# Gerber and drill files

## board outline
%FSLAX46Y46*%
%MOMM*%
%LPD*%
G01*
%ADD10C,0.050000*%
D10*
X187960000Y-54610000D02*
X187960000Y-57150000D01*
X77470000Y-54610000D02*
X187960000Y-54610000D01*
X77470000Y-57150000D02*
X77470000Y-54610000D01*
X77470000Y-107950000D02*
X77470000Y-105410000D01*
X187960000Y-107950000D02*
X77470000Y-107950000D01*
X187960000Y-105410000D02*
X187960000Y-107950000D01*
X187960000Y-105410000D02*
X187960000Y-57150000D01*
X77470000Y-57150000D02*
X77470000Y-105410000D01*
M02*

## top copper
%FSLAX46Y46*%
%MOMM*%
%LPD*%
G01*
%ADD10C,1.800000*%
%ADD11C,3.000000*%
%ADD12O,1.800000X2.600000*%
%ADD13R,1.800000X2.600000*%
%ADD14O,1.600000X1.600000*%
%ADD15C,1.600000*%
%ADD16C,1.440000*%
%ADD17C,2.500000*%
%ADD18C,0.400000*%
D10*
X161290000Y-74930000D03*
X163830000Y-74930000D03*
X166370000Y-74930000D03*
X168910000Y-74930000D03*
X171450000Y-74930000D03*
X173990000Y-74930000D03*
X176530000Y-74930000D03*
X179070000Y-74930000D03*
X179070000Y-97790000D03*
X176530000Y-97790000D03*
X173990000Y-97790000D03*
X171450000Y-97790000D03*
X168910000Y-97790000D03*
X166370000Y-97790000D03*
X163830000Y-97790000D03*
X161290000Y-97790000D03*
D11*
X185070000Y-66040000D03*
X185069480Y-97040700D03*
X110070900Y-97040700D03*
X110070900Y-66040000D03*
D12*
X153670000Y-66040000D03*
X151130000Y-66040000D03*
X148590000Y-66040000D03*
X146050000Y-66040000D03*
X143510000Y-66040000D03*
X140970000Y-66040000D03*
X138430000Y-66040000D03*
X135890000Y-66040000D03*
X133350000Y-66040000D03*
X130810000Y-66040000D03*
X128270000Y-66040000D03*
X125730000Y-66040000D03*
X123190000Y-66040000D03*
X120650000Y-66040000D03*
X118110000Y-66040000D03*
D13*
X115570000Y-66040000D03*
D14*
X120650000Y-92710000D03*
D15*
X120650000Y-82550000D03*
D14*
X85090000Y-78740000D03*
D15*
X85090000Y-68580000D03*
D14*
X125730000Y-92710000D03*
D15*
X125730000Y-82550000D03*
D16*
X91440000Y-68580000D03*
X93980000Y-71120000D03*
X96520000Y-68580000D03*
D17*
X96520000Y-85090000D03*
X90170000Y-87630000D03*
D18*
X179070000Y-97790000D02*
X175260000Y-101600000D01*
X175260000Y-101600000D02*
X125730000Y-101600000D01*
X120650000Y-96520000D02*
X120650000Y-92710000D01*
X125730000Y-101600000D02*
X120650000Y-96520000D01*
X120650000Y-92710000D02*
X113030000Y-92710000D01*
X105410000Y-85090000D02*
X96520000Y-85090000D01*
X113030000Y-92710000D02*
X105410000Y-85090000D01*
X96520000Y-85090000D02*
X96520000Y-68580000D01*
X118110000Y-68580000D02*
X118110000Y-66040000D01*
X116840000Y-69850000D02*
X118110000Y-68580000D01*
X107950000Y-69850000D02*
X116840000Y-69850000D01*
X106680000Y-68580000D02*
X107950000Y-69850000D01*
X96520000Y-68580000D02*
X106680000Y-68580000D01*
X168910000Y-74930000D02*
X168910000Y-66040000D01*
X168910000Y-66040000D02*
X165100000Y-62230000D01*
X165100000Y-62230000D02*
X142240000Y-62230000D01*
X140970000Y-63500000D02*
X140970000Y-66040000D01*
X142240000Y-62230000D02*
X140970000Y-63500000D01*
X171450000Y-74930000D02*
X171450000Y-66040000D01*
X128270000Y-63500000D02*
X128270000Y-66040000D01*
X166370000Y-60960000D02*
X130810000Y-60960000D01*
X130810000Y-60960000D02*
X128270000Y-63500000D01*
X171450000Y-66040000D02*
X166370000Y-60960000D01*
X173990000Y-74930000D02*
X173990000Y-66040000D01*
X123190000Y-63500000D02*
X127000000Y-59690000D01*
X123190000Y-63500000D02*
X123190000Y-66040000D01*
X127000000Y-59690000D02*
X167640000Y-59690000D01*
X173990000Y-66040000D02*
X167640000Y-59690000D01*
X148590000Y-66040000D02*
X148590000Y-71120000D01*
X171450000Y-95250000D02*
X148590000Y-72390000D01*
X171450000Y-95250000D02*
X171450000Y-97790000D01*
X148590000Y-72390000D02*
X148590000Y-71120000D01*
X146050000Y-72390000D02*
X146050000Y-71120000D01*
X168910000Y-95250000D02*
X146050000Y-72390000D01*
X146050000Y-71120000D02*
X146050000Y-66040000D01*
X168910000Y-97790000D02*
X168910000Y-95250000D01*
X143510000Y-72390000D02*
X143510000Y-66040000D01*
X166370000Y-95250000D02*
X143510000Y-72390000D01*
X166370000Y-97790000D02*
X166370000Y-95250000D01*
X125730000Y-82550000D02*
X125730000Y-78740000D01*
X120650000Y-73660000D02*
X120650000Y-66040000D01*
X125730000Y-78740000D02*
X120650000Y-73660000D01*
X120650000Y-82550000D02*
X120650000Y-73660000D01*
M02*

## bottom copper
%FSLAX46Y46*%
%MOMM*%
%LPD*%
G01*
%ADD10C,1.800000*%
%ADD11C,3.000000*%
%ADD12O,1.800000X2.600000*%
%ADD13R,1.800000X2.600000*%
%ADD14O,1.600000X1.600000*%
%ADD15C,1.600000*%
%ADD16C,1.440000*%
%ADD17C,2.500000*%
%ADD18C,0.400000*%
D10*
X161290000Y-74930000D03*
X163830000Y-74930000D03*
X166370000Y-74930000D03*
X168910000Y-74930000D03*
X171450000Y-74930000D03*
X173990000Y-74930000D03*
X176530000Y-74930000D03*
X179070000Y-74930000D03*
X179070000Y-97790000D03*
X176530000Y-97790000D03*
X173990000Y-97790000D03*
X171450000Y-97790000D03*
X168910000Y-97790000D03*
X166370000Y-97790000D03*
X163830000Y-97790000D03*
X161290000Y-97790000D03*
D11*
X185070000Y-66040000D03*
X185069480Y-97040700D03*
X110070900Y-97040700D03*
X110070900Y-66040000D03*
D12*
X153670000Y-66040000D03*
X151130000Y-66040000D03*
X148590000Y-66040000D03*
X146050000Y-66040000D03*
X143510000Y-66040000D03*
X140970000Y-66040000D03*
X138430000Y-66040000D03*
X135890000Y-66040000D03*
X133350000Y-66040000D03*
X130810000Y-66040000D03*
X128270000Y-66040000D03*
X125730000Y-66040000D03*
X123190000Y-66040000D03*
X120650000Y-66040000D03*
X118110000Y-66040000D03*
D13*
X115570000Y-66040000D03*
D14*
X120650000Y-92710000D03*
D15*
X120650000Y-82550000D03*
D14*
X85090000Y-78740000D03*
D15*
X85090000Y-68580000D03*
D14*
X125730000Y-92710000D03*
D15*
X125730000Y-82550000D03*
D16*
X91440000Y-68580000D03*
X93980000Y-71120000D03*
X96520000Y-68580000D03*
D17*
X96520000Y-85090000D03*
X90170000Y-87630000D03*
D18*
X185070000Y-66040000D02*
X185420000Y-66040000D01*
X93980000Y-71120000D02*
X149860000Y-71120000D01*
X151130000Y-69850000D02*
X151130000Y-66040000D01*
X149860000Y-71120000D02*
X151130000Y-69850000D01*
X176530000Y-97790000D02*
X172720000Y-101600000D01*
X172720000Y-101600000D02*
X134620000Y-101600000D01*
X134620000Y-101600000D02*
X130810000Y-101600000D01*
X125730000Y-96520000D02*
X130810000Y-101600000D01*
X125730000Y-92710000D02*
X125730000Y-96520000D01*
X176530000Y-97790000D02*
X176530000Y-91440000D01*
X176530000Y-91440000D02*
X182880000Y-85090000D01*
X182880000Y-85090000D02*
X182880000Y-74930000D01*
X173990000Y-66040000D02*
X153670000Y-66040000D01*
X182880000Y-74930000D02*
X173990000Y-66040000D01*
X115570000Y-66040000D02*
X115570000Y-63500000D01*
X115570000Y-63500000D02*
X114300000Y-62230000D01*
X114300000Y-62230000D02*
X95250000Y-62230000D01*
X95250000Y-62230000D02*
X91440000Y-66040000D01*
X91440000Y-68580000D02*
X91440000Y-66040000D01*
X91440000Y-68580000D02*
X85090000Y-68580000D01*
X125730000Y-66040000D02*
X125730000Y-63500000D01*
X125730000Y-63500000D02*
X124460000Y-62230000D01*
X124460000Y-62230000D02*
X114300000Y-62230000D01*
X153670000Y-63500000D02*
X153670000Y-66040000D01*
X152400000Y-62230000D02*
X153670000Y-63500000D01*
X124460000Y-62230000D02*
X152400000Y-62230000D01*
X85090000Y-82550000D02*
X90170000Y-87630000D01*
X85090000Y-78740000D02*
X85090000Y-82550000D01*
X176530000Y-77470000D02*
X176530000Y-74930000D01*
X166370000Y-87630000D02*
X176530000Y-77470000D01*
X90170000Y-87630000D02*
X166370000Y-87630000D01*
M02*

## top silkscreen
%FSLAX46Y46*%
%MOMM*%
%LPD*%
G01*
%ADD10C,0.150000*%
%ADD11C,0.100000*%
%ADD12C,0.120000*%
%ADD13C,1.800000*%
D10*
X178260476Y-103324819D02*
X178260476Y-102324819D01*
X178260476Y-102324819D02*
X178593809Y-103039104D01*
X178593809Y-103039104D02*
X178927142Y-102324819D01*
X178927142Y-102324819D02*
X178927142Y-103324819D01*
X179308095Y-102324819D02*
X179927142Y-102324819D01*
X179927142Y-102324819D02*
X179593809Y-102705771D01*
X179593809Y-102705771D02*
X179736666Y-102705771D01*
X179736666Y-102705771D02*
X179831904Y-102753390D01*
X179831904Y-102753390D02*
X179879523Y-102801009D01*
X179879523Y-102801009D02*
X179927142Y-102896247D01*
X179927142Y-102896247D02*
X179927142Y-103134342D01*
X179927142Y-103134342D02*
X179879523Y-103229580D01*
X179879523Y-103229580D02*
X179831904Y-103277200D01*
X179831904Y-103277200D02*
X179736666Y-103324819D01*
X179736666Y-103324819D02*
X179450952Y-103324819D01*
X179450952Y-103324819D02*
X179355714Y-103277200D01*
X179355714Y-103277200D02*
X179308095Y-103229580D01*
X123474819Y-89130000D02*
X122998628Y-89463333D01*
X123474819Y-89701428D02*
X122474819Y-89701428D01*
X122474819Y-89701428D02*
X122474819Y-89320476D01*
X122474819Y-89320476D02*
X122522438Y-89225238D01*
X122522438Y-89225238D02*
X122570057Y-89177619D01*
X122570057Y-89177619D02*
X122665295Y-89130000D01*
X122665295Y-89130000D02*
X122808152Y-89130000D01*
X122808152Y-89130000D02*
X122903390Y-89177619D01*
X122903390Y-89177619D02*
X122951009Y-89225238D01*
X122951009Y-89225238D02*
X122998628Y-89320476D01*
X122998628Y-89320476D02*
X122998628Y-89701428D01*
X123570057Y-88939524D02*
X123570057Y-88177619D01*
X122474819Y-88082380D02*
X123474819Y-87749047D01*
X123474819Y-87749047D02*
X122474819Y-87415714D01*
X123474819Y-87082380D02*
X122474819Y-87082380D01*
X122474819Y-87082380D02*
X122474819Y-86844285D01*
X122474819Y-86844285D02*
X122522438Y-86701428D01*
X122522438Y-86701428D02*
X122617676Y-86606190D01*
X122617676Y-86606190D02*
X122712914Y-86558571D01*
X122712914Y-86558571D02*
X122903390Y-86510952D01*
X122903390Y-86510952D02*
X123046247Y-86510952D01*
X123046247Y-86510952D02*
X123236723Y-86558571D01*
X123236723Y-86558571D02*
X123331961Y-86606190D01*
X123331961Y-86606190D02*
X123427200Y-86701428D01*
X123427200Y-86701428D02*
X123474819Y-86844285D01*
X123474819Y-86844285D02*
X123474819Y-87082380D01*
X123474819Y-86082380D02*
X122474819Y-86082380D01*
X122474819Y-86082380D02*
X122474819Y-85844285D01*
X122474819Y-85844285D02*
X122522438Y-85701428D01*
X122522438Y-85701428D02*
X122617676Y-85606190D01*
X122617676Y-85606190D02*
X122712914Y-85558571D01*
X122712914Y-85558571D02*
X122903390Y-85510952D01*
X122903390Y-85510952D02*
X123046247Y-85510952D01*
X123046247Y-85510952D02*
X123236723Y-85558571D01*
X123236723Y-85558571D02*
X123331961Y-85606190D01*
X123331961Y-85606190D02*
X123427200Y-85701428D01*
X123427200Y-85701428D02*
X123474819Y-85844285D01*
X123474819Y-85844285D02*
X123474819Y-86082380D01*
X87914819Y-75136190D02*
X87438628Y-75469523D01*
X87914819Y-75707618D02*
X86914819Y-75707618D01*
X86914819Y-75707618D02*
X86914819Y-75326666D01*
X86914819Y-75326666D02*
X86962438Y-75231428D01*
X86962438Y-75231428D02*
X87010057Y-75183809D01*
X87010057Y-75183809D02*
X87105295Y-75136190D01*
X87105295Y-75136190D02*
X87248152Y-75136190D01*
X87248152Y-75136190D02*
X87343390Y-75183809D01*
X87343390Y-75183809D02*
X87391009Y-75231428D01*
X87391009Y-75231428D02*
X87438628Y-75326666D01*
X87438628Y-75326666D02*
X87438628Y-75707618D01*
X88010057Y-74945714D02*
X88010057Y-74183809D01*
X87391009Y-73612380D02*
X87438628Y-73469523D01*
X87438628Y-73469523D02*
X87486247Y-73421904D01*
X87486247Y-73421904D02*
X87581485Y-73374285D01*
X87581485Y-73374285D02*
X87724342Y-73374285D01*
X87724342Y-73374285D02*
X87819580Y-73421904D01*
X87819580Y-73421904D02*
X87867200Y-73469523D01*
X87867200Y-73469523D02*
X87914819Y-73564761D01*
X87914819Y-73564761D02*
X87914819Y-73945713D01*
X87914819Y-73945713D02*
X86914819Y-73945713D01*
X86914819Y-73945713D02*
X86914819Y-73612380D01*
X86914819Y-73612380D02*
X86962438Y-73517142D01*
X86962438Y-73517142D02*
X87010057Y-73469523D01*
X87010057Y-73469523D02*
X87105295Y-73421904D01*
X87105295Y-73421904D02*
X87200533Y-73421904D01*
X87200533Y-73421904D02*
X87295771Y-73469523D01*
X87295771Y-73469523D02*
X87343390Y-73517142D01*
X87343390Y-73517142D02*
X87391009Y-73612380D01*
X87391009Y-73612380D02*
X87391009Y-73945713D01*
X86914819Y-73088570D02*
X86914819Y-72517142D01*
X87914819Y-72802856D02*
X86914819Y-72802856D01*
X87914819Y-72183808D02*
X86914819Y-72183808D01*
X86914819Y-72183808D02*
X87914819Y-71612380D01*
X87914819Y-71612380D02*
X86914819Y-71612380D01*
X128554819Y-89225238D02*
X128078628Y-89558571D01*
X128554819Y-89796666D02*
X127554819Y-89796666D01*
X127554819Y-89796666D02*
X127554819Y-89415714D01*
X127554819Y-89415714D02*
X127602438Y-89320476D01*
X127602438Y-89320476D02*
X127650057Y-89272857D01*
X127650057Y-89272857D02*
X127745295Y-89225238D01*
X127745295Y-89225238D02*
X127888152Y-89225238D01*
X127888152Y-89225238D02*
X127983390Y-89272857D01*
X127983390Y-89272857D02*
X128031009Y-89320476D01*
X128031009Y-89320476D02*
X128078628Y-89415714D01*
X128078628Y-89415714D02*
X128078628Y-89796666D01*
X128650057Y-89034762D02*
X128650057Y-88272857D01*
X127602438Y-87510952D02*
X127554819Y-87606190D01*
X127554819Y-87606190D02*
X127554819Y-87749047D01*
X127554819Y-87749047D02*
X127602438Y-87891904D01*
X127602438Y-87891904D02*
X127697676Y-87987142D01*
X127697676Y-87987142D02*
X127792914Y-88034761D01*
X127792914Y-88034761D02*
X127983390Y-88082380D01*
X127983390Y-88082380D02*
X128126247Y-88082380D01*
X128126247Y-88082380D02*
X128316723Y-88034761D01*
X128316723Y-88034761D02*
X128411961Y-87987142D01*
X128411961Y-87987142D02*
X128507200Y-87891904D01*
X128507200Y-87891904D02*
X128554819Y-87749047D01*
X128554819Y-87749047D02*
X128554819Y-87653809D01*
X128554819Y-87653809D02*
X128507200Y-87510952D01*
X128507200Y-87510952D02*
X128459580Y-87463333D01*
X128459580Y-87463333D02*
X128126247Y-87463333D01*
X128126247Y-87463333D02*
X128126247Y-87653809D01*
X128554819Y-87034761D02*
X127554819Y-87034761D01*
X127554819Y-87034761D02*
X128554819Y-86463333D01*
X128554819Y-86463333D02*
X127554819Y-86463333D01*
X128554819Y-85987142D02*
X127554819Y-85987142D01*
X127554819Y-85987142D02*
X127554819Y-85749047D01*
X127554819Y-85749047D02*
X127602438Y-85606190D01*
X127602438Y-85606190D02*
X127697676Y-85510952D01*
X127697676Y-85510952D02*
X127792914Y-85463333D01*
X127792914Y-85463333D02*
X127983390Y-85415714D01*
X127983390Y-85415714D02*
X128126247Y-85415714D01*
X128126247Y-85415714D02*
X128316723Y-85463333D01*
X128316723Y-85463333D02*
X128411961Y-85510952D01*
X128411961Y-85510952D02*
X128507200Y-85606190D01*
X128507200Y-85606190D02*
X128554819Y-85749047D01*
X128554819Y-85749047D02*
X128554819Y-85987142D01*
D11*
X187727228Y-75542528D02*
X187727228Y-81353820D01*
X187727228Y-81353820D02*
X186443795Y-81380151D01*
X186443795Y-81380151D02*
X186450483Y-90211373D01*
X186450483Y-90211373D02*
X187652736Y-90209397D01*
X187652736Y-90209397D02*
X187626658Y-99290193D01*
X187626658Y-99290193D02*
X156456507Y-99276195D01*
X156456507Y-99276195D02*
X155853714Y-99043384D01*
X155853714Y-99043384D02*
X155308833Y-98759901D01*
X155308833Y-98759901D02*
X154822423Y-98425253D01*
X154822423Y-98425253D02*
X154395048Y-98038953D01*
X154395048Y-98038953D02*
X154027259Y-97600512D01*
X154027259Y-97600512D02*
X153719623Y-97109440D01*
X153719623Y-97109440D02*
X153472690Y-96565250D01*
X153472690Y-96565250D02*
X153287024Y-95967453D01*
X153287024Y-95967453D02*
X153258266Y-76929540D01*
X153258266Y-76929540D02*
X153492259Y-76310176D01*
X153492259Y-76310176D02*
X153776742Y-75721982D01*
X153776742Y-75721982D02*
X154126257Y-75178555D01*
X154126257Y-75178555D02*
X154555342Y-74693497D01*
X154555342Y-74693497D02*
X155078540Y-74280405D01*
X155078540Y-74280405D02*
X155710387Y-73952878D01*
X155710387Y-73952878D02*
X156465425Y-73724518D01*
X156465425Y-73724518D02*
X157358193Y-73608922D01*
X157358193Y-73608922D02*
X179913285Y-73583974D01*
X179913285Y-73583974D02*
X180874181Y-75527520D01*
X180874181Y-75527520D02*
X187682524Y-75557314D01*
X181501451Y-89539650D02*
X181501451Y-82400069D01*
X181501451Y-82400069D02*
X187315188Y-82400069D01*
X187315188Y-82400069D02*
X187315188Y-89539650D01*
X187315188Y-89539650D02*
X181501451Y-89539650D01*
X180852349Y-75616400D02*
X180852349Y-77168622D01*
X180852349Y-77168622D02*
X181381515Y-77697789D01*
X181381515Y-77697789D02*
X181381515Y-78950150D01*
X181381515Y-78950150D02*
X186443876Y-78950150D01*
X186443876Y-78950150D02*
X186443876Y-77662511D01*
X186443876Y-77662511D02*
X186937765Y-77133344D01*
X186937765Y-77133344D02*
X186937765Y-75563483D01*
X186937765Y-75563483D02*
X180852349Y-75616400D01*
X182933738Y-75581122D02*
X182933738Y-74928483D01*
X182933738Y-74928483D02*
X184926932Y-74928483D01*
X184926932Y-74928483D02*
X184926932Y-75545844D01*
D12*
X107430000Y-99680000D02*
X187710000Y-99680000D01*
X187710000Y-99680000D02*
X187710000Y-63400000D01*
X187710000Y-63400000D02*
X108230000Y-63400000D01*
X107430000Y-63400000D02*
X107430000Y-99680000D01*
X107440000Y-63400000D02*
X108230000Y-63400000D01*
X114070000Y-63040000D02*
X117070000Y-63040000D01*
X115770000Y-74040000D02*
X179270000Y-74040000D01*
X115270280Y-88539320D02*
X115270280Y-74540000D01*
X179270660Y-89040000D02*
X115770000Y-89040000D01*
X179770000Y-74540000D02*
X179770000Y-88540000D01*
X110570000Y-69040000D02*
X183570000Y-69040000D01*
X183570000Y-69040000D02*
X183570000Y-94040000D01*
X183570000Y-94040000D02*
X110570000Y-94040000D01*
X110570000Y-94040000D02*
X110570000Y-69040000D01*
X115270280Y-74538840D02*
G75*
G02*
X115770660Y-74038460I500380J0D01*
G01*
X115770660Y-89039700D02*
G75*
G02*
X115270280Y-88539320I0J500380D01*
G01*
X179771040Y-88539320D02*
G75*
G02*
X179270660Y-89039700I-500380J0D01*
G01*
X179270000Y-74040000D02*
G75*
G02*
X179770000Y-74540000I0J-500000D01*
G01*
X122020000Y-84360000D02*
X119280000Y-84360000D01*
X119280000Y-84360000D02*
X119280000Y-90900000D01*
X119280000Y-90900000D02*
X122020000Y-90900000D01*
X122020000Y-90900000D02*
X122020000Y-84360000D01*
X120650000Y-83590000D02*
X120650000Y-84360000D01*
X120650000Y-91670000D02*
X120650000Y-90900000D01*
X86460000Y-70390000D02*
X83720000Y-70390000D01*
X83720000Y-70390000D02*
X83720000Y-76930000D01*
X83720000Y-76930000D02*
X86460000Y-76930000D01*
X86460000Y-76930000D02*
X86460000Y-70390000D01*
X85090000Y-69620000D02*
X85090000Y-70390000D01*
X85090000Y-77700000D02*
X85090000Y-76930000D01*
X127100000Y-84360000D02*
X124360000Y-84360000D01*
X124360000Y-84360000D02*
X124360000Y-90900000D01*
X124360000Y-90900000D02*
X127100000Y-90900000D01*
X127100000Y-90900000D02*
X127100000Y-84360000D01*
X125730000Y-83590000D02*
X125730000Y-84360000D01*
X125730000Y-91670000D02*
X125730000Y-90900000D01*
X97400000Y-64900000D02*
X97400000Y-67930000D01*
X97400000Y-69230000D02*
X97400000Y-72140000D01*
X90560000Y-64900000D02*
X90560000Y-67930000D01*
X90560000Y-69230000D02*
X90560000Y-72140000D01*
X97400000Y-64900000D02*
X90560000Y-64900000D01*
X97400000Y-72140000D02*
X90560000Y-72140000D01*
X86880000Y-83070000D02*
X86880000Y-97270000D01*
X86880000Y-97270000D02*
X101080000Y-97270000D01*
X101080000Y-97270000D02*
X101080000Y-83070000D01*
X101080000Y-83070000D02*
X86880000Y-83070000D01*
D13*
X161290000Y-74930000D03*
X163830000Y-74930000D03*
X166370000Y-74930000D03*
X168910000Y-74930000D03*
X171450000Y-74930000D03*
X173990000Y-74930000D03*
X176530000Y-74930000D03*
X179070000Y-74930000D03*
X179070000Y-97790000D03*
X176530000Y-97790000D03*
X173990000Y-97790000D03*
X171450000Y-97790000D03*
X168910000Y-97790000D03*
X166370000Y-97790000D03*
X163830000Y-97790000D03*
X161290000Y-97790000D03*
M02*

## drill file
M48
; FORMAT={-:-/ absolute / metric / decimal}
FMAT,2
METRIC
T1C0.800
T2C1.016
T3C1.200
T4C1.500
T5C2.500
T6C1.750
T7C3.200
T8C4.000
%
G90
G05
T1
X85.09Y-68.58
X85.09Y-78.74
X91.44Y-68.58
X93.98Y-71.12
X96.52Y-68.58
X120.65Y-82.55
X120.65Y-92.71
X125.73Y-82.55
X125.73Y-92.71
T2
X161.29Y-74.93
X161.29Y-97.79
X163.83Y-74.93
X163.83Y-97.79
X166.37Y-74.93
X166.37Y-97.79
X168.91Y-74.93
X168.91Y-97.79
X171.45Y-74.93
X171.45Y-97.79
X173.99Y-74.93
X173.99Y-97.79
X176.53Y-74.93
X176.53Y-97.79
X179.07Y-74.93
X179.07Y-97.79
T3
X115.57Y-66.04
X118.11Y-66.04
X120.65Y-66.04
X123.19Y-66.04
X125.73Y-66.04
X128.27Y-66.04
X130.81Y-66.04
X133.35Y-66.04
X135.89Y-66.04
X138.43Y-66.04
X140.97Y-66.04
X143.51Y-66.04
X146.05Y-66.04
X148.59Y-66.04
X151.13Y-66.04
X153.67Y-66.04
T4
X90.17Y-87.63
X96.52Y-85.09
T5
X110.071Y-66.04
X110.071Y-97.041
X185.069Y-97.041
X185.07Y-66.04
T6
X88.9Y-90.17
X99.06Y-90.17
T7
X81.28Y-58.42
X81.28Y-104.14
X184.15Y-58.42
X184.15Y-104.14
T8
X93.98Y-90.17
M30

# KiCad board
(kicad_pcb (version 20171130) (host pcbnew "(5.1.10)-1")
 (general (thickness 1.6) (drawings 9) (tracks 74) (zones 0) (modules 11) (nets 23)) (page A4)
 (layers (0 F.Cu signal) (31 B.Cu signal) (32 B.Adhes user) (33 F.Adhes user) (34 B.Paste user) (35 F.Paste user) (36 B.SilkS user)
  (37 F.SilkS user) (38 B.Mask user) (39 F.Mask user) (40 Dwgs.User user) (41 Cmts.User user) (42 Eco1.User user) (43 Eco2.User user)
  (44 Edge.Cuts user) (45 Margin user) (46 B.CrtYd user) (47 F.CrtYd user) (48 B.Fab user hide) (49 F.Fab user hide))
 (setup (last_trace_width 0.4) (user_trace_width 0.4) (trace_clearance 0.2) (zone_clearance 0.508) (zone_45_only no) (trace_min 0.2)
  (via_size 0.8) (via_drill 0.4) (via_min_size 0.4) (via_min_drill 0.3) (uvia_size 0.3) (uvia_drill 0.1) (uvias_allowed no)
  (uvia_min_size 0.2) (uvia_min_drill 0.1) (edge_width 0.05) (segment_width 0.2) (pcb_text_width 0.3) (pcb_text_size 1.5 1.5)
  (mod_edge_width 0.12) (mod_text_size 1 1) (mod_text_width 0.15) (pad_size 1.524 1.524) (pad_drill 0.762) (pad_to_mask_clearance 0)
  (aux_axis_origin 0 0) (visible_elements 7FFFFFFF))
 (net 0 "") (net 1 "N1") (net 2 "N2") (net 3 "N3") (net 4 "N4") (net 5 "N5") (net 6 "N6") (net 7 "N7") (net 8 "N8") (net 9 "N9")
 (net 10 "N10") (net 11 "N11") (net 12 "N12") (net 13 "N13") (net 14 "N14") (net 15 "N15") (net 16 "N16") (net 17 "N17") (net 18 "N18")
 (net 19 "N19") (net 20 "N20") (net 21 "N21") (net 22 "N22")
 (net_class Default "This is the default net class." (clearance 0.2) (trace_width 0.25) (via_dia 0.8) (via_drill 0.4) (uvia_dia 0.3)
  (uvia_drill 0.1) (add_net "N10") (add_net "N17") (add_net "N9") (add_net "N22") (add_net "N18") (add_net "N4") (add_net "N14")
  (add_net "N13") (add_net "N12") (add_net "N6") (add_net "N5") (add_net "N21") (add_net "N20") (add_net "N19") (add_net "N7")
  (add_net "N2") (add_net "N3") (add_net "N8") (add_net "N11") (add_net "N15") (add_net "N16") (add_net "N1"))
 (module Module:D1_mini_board (layer F.Cu) (at 171.45 86.36 90)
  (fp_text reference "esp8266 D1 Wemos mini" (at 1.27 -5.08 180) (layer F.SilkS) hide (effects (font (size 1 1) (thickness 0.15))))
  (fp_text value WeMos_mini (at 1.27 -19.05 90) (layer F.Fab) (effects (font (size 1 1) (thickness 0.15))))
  (fp_line (start 10.817472 16.277228) (end 5.00618 16.277228) (layer F.SilkS) (width 0.1))
  (fp_line (start 5.00618 16.277228) (end 4.979849 14.993795) (layer F.SilkS) (width 0.1))
  (fp_line (start 4.979849 14.993795) (end -3.851373 15.000483) (layer F.SilkS) (width 0.1))
  (fp_line (start -3.851373 15.000483) (end -3.849397 16.202736) (layer F.SilkS) (width 0.1))
  (fp_line (start -3.849397 16.202736) (end -12.930193 16.176658) (layer F.SilkS) (width 0.1))
  (fp_line (start -12.930193 16.176658) (end -12.916195 -14.993493) (layer F.SilkS) (width 0.1))
  (fp_line (start -12.916195 -14.993493) (end -12.683384 -15.596286) (layer F.SilkS) (width 0.1))
  (fp_line (start -12.683384 -15.596286) (end -12.399901 -16.141167) (layer F.SilkS) (width 0.1))
  (fp_line (start -12.399901 -16.141167) (end -12.065253 -16.627577) (layer F.SilkS) (width 0.1))
  (fp_line (start -12.065253 -16.627577) (end -11.678953 -17.054952) (layer F.SilkS) (width 0.1))
  (fp_line (start -11.678953 -17.054952) (end -11.240512 -17.422741) (layer F.SilkS) (width 0.1))
  (fp_line (start -11.240512 -17.422741) (end -10.74944 -17.730377) (layer F.SilkS) (width 0.1))
  (fp_line (start -10.74944 -17.730377) (end -10.20525 -17.97731) (layer F.SilkS) (width 0.1))
  (fp_line (start -10.20525 -17.97731) (end -9.607453 -18.162976) (layer F.SilkS) (width 0.1))
  (fp_line (start -9.607453 -18.162976) (end 9.43046 -18.191734) (layer F.SilkS) (width 0.1))
  (fp_line (start 9.43046 -18.191734) (end 10.049824 -17.957741) (layer F.SilkS) (width 0.1))
  (fp_line (start 10.049824 -17.957741) (end 10.638018 -17.673258) (layer F.SilkS) (width 0.1))
  (fp_line (start 10.638018 -17.673258) (end 11.181445 -17.323743) (layer F.SilkS) (width 0.1))
  (fp_line (start 11.181445 -17.323743) (end 11.666503 -16.894658) (layer F.SilkS) (width 0.1))
  (fp_line (start 11.666503 -16.894658) (end 12.079595 -16.37146) (layer F.SilkS) (width 0.1))
  (fp_line (start 12.079595 -16.37146) (end 12.407122 -15.739613) (layer F.SilkS) (width 0.1))
  (fp_line (start 12.407122 -15.739613) (end 12.635482 -14.984575) (layer F.SilkS) (width 0.1))
  (fp_line (start 12.635482 -14.984575) (end 12.751078 -14.091807) (layer F.SilkS) (width 0.1))
  (fp_line (start 12.751078 -14.091807) (end 12.776026 8.463285) (layer F.SilkS) (width 0.1))
  (fp_line (start 12.776026 8.463285) (end 10.83248 9.424181) (layer F.SilkS) (width 0.1))
  (fp_line (start 10.83248 9.424181) (end 10.802686 16.232524) (layer F.SilkS) (width 0.1))
  (fp_line (start -3.17965 10.051451) (end 3.959931 10.051451) (layer F.SilkS) (width 0.1))
  (fp_line (start 3.959931 10.051451) (end 3.959931 15.865188) (layer F.SilkS) (width 0.1))
  (fp_line (start 3.959931 15.865188) (end -3.17965 15.865188) (layer F.SilkS) (width 0.1))
  (fp_line (start -3.17965 15.865188) (end -3.17965 10.051451) (layer F.SilkS) (width 0.1))
  (fp_line (start 10.7436 9.402349) (end 9.191378 9.402349) (layer F.SilkS) (width 0.1))
  (fp_line (start 9.191378 9.402349) (end 8.662211 9.931515) (layer F.SilkS) (width 0.1))
  (fp_line (start 8.662211 9.931515) (end 7.40985 9.931515) (layer F.SilkS) (width 0.1))
  (fp_line (start 7.40985 9.931515) (end 7.40985 14.993876) (layer F.SilkS) (width 0.1))
  (fp_line (start 7.40985 14.993876) (end 8.697489 14.993876) (layer F.SilkS) (width 0.1))
  (fp_line (start 8.697489 14.993876) (end 9.226656 15.487765) (layer F.SilkS) (width 0.1))
  (fp_line (start 9.226656 15.487765) (end 10.796517 15.487765) (layer F.SilkS) (width 0.1))
  (fp_line (start 10.796517 15.487765) (end 10.7436 9.402349) (layer F.SilkS) (width 0.1))
  (fp_line (start 10.778878 11.483738) (end 11.431517 11.483738) (layer F.SilkS) (width 0.1))
  (fp_line (start 11.431517 11.483738) (end 11.431517 13.476932) (layer F.SilkS) (width 0.1))
  (fp_line (start 11.431517 13.476932) (end 10.814156 13.476932) (layer F.SilkS) (width 0.1))
  (pad 9 thru_hole circle (at 11.43 -10.16 90) (size 1.8 1.8) (drill 1.016) (layers *.Cu *.Mask F.SilkS) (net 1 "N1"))
  (pad 10 thru_hole circle (at 11.43 -7.62 90) (size 1.8 1.8) (drill 1.016) (layers *.Cu *.Mask F.SilkS) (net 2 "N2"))
  (pad 11 thru_hole circle (at 11.43 -5.08 90) (size 1.8 1.8) (drill 1.016) (layers *.Cu *.Mask F.SilkS) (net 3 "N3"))
  (pad 12 thru_hole circle (at 11.43 -2.54 90) (size 1.8 1.8) (drill 1.016) (layers *.Cu *.Mask F.SilkS) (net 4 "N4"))
  (pad 13 thru_hole circle (at 11.43 0 90) (size 1.8 1.8) (drill 1.016) (layers *.Cu *.Mask F.SilkS) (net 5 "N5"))
  (pad 14 thru_hole circle (at 11.43 2.54 90) (size 1.8 1.8) (drill 1.016) (layers *.Cu *.Mask F.SilkS) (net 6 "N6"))
  (pad 15 thru_hole circle (at 11.43 5.08 90) (size 1.8 1.8) (drill 1.016) (layers *.Cu *.Mask F.SilkS) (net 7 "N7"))
  (pad 16 thru_hole circle (at 11.43 7.62 90) (size 1.8 1.8) (drill 1.016) (layers *.Cu *.Mask F.SilkS) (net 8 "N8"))
  (pad 1 thru_hole circle (at -11.43 7.62 90) (size 1.8 1.8) (drill 1.016) (layers *.Cu *.Mask F.SilkS) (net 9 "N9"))
  (pad 2 thru_hole circle (at -11.43 5.08 90) (size 1.8 1.8) (drill 1.016) (layers *.Cu *.Mask F.SilkS) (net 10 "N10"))
  (pad 3 thru_hole circle (at -11.43 2.54 90) (size 1.8 1.8) (drill 1.016) (layers *.Cu *.Mask F.SilkS) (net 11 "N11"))
  (pad 4 thru_hole circle (at -11.43 0 90) (size 1.8 1.8) (drill 1.016) (layers *.Cu *.Mask F.SilkS) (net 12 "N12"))
  (pad 5 thru_hole circle (at -11.43 -2.54 90) (size 1.8 1.8) (drill 1.016) (layers *.Cu *.Mask F.SilkS) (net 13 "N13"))
  (pad 6 thru_hole circle (at -11.43 -5.08 90) (size 1.8 1.8) (drill 1.016) (layers *.Cu *.Mask F.SilkS) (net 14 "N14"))
  (pad 7 thru_hole circle (at -11.43 -7.62 90) (size 1.8 1.8) (drill 1.016) (layers *.Cu *.Mask F.SilkS) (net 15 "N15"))
  (pad 8 thru_hole circle (at -11.43 -10.16 90) (size 1.8 1.8) (drill 1.016) (layers *.Cu *.Mask F.SilkS) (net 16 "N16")))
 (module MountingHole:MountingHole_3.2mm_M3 (layer F.Cu) (at 184.15 104.14)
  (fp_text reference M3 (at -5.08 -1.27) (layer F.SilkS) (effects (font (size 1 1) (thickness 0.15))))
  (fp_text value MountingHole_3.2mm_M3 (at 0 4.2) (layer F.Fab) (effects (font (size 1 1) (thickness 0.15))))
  (pad 1 np_thru_hole circle (at 0 0) (size 3.2 3.2) (drill 3.2) (layers *.Cu *.Mask)))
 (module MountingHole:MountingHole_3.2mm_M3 (layer F.Cu) (at 81.28 104.14)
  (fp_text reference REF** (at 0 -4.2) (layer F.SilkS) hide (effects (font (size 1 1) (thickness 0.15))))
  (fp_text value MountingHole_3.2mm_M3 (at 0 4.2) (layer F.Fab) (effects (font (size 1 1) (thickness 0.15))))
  (pad 1 np_thru_hole circle (at 0 0) (size 3.2 3.2) (drill 3.2) (layers *.Cu *.Mask)))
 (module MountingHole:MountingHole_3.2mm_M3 (layer F.Cu) (at 81.28 58.42)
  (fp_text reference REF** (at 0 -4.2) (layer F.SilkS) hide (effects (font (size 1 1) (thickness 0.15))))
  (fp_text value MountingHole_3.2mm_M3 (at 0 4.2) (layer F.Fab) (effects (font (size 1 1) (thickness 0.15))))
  (pad 1 np_thru_hole circle (at 0 0) (size 3.2 3.2) (drill 3.2) (layers *.Cu *.Mask)))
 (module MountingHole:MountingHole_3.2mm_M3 (layer F.Cu) (at 184.15 58.42)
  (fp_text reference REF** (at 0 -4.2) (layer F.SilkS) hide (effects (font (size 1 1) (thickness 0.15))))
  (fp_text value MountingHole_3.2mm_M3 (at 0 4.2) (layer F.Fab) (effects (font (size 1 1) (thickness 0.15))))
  (pad 1 np_thru_hole circle (at 0 0) (size 3.2 3.2) (drill 3.2) (layers *.Cu *.Mask)))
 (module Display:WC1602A (layer F.Cu) (at 115.57 66.04)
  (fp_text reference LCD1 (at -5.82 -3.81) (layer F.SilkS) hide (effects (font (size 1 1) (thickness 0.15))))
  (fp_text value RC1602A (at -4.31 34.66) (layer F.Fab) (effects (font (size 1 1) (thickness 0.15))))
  (fp_line (start -8.14 33.64) (end 72.14 33.64) (layer F.SilkS) (width 0.12))
  (fp_line (start 72.14 33.64) (end 72.14 -2.64) (layer F.SilkS) (width 0.12))
  (fp_line (start 72.14 -2.64) (end -7.34 -2.64) (layer F.SilkS) (width 0.12))
  (fp_line (start -8.14 -2.64) (end -8.14 33.64) (layer F.SilkS) (width 0.12))
  (fp_line (start -8.13 -2.64) (end -7.34 -2.64) (layer F.SilkS) (width 0.12))
  (fp_line (start -1.5 -3) (end 1.5 -3) (layer F.SilkS) (width 0.12))
  (fp_line (start 0.2 8) (end 63.7 8) (layer F.SilkS) (width 0.12))
  (fp_line (start -0.29972 22.49932) (end -0.29972 8.5) (layer F.SilkS) (width 0.12))
  (fp_line (start 63.70066 23) (end 0.2 23) (layer F.SilkS) (width 0.12))
  (fp_line (start 64.2 8.5) (end 64.2 22.5) (layer F.SilkS) (width 0.12))
  (fp_line (start -5 3) (end 68 3) (layer F.SilkS) (width 0.12))
  (fp_line (start 68 3) (end 68 28) (layer F.SilkS) (width 0.12))
  (fp_line (start 68 28) (end -5 28) (layer F.SilkS) (width 0.12))
  (fp_line (start -5 28) (end -5 3) (layer F.SilkS) (width 0.12))
  (fp_arc (start 0.20066 8.49884) (end -0.29972 8.49884) (angle 90) (layer F.SilkS) (width 0.12))
  (fp_arc (start 0.20066 22.49932) (end 0.20066 22.9997) (angle 90) (layer F.SilkS) (width 0.12))
  (fp_arc (start 63.70066 22.49932) (end 64.20104 22.49932) (angle 90) (layer F.SilkS) (width 0.12))
  (fp_arc (start 63.7 8.5) (end 63.7 8) (angle 90) (layer F.SilkS) (width 0.12))
  (pad "" thru_hole circle (at 69.5 0) (size 3 3) (drill 2.5) (layers *.Cu *.Mask))
  (pad "" thru_hole circle (at 69.49948 31.0007) (size 3 3) (drill 2.5) (layers *.Cu *.Mask))
  (pad "" thru_hole circle (at -5.4991 31.0007) (size 3 3) (drill 2.5) (layers *.Cu *.Mask))
  (pad "" thru_hole circle (at -5.4991 0) (size 3 3) (drill 2.5) (layers *.Cu *.Mask))
  (pad 16 thru_hole oval (at 38.1 0) (size 1.8 2.6) (drill 1.2) (layers *.Cu *.Mask) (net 10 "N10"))
  (pad 15 thru_hole oval (at 35.56 0) (size 1.8 2.6) (drill 1.2) (layers *.Cu *.Mask) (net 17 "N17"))
  (pad 14 thru_hole oval (at 33.02 0) (size 1.8 2.6) (drill 1.2) (layers *.Cu *.Mask) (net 12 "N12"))
  (pad 13 thru_hole oval (at 30.48 0) (size 1.8 2.6) (drill 1.2) (layers *.Cu *.Mask) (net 13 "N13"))
  (pad 12 thru_hole oval (at 27.94 0) (size 1.8 2.6) (drill 1.2) (layers *.Cu *.Mask) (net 14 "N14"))
  (pad 11 thru_hole oval (at 25.4 0) (size 1.8 2.6) (drill 1.2) (layers *.Cu *.Mask) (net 4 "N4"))
  (pad 10 thru_hole oval (at 22.86 0) (size 1.8 2.6) (drill 1.2) (layers *.Cu *.Mask) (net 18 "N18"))
  (pad 9 thru_hole oval (at 20.32 0) (size 1.8 2.6) (drill 1.2) (layers *.Cu *.Mask) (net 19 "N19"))
  (pad 8 thru_hole oval (at 17.78 0) (size 1.8 2.6) (drill 1.2) (layers *.Cu *.Mask) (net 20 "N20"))
  (pad 7 thru_hole oval (at 15.24 0) (size 1.8 2.6) (drill 1.2) (layers *.Cu *.Mask) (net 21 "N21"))
  (pad 6 thru_hole oval (at 12.7 0) (size 1.8 2.6) (drill 1.2) (layers *.Cu *.Mask) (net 5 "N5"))
  (pad 5 thru_hole oval (at 10.16 0) (size 1.8 2.6) (drill 1.2) (layers *.Cu *.Mask) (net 10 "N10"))
  (pad 4 thru_hole oval (at 7.62 0) (size 1.8 2.6) (drill 1.2) (layers *.Cu *.Mask) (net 6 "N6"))
  (pad 3 thru_hole oval (at 5.08 0) (size 1.8 2.6) (drill 1.2) (layers *.Cu *.Mask) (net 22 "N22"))
  (pad 2 thru_hole oval (at 2.54 0) (size 1.8 2.6) (drill 1.2) (layers *.Cu *.Mask) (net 9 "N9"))
  (pad 1 thru_hole rect (at 0 0) (size 1.8 2.6) (drill 1.2) (layers *.Cu *.Mask) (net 10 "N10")))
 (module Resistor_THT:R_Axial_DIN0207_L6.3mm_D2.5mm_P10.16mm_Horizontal (layer F.Cu) (at 120.65 82.55 270)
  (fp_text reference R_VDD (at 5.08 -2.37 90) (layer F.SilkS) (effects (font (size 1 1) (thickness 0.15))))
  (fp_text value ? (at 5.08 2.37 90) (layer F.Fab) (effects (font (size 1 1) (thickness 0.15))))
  (fp_line (start 1.81 -1.37) (end 1.81 1.37) (layer F.SilkS) (width 0.12))
  (fp_line (start 1.81 1.37) (end 8.35 1.37) (layer F.SilkS) (width 0.12))
  (fp_line (start 8.35 1.37) (end 8.35 -1.37) (layer F.SilkS) (width 0.12))
  (fp_line (start 8.35 -1.37) (end 1.81 -1.37) (layer F.SilkS) (width 0.12))
  (fp_line (start 1.04 0) (end 1.81 0) (layer F.SilkS) (width 0.12))
  (fp_line (start 9.12 0) (end 8.35 0) (layer F.SilkS) (width 0.12))
  (pad 2 thru_hole oval (at 10.16 0 270) (size 1.6 1.6) (drill 0.8) (layers *.Cu *.Mask) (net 9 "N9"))
  (pad 1 thru_hole circle (at 0 0 270) (size 1.6 1.6) (drill 0.8) (layers *.Cu *.Mask) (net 22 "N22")))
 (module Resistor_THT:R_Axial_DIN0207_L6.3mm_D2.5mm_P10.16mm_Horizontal (layer F.Cu) (at 85.09 68.58 270)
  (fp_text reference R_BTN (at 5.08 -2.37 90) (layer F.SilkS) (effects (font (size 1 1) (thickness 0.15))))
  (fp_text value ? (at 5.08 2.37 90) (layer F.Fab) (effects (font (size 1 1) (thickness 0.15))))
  (fp_line (start 1.81 -1.37) (end 1.81 1.37) (layer F.SilkS) (width 0.12))
  (fp_line (start 1.81 1.37) (end 8.35 1.37) (layer F.SilkS) (width 0.12))
  (fp_line (start 8.35 1.37) (end 8.35 -1.37) (layer F.SilkS) (width 0.12))
  (fp_line (start 8.35 -1.37) (end 1.81 -1.37) (layer F.SilkS) (width 0.12))
  (fp_line (start 1.04 0) (end 1.81 0) (layer F.SilkS) (width 0.12))
  (fp_line (start 9.12 0) (end 8.35 0) (layer F.SilkS) (width 0.12))
  (pad 2 thru_hole oval (at 10.16 0 270) (size 1.6 1.6) (drill 0.8) (layers *.Cu *.Mask) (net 7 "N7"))
  (pad 1 thru_hole circle (at 0 0 270) (size 1.6 1.6) (drill 0.8) (layers *.Cu *.Mask) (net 10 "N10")))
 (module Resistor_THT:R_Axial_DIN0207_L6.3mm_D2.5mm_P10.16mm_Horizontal (layer F.Cu) (at 125.73 82.55 270)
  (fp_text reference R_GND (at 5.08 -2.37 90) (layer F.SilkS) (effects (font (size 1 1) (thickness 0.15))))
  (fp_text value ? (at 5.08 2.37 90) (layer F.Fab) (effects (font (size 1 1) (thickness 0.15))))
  (fp_line (start 1.81 -1.37) (end 1.81 1.37) (layer F.SilkS) (width 0.12))
  (fp_line (start 1.81 1.37) (end 8.35 1.37) (layer F.SilkS) (width 0.12))
  (fp_line (start 8.35 1.37) (end 8.35 -1.37) (layer F.SilkS) (width 0.12))
  (fp_line (start 8.35 -1.37) (end 1.81 -1.37) (layer F.SilkS) (width 0.12))
  (fp_line (start 1.04 0) (end 1.81 0) (layer F.SilkS) (width 0.12))
  (fp_line (start 9.12 0) (end 8.35 0) (layer F.SilkS) (width 0.12))
  (pad 2 thru_hole oval (at 10.16 0 270) (size 1.6 1.6) (drill 0.8) (layers *.Cu *.Mask) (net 10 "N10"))
  (pad 1 thru_hole circle (at 0 0 270) (size 1.6 1.6) (drill 0.8) (layers *.Cu *.Mask) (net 22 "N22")))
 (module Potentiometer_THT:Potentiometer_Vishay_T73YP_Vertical (layer F.Cu) (at 91.44 68.58 270)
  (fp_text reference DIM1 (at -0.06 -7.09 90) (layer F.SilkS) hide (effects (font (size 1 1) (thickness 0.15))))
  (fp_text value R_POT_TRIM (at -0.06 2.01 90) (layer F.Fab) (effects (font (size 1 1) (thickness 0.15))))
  (fp_line (start -3.68 -5.96) (end -0.65 -5.96) (layer F.SilkS) (width 0.12))
  (fp_line (start 0.65 -5.96) (end 3.56 -5.96) (layer F.SilkS) (width 0.12))
  (fp_line (start -3.68 0.88) (end -0.65 0.88) (layer F.SilkS) (width 0.12))
  (fp_line (start 0.65 0.88) (end 3.56 0.88) (layer F.SilkS) (width 0.12))
  (fp_line (start -3.68 -5.96) (end -3.68 0.88) (layer F.SilkS) (width 0.12))
  (fp_line (start 3.56 -5.96) (end 3.56 0.88) (layer F.SilkS) (width 0.12))
  (pad 1 thru_hole circle (at 0 0 270) (size 1.44 1.44) (drill 0.8) (layers *.Cu *.Mask) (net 10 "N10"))
  (pad 2 thru_hole circle (at 2.54 -2.54 270) (size 1.44 1.44) (drill 0.8) (layers *.Cu *.Mask) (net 17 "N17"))
  (pad 3 thru_hole circle (at 0 -5.08 270) (size 1.44 1.44) (drill 0.8) (layers *.Cu *.Mask) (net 9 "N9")))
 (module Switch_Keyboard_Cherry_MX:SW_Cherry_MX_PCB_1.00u (layer F.Cu) (at 93.98 90.17)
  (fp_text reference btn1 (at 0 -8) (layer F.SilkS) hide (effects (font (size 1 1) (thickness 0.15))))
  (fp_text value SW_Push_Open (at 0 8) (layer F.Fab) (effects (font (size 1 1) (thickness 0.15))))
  (fp_line (start -7.1 -7.1) (end -7.1 7.1) (layer F.SilkS) (width 0.12))
  (fp_line (start -7.1 7.1) (end 7.1 7.1) (layer F.SilkS) (width 0.12))
  (fp_line (start 7.1 7.1) (end 7.1 -7.1) (layer F.SilkS) (width 0.12))
  (fp_line (start 7.1 -7.1) (end -7.1 -7.1) (layer F.SilkS) (width 0.12))
  (pad "" np_thru_hole circle (at 5.08 0) (size 1.75 1.75) (drill 1.75) (layers *.Cu *.Mask))
  (pad "" np_thru_hole circle (at -5.08 0) (size 1.75 1.75) (drill 1.75) (layers *.Cu *.Mask))
  (pad "" np_thru_hole circle (at 0 0) (size 4 4) (drill 4) (layers *.Cu *.Mask))
  (pad 2 thru_hole circle (at 2.54 -5.08) (size 2.5 2.5) (drill 1.5) (layers *.Cu B.Mask) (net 9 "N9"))
  (pad 1 thru_hole circle (at -3.81 -2.54) (size 2.5 2.5) (drill 1.5) (layers *.Cu B.Mask) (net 7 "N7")))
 (gr_line (start 187.96 54.61) (end 187.96 57.15) (layer Edge.Cuts) (width 0.05))
 (gr_line (start 77.47 54.61) (end 187.96 54.61) (layer Edge.Cuts) (width 0.05))
 (gr_line (start 77.47 57.15) (end 77.47 54.61) (layer Edge.Cuts) (width 0.05))
 (gr_line (start 77.47 107.95) (end 77.47 105.41) (layer Edge.Cuts) (width 0.05))
 (gr_line (start 187.96 107.95) (end 77.47 107.95) (layer Edge.Cuts) (width 0.05))
 (gr_line (start 187.96 105.41) (end 187.96 107.95) (layer Edge.Cuts) (width 0.05))
 (gr_line (start 187.96 105.41) (end 187.96 57.15) (layer Edge.Cuts) (width 0.05))
 (gr_line (start 77.47 57.15) (end 77.47 105.41) (layer Edge.Cuts) (width 0.05))
 (segment (start 185.07 66.04) (end 185.42 66.04) (width 0.4) (layer B.Cu) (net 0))
 (segment (start 179.07 97.79) (end 175.26 101.6) (width 0.4) (layer F.Cu) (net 9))
 (segment (start 175.26 101.6) (end 125.73 101.6) (width 0.4) (layer F.Cu) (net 9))
 (segment (start 120.65 96.52) (end 120.65 92.71) (width 0.4) (layer F.Cu) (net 9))
 (segment (start 125.73 101.6) (end 120.65 96.52) (width 0.4) (layer F.Cu) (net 9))
 (segment (start 120.65 92.71) (end 113.03 92.71) (width 0.4) (layer F.Cu) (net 9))
 (segment (start 105.41 85.09) (end 96.52 85.09) (width 0.4) (layer F.Cu) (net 9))
 (segment (start 113.03 92.71) (end 105.41 85.09) (width 0.4) (layer F.Cu) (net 9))
 (segment (start 96.52 85.09) (end 96.52 68.58) (width 0.4) (layer F.Cu) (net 9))
 (segment (start 118.11 68.58) (end 118.11 66.04) (width 0.4) (layer F.Cu) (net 9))
 (segment (start 116.84 69.85) (end 118.11 68.58) (width 0.4) (layer F.Cu) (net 9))
 (segment (start 107.95 69.85) (end 116.84 69.85) (width 0.4) (layer F.Cu) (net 9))
 (segment (start 106.68 68.58) (end 107.95 69.85) (width 0.4) (layer F.Cu) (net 9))
 (segment (start 96.52 68.58) (end 106.68 68.58) (width 0.4) (layer F.Cu) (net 9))
 (segment (start 93.98 71.12) (end 149.86 71.12) (width 0.4) (layer B.Cu) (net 17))
 (segment (start 151.13 69.85) (end 151.13 66.04) (width 0.4) (layer B.Cu) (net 17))
 (segment (start 149.86 71.12) (end 151.13 69.85) (width 0.4) (layer B.Cu) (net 17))
 (segment (start 176.53 97.79) (end 172.72 101.6) (width 0.4) (layer B.Cu) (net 10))
 (segment (start 172.72 101.6) (end 134.62 101.6) (width 0.4) (layer B.Cu) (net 10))
 (segment (start 134.62 101.6) (end 130.81 101.6) (width 0.4) (layer B.Cu) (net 10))
 (segment (start 125.73 96.52) (end 130.81 101.6) (width 0.4) (layer B.Cu) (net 10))
 (segment (start 125.73 92.71) (end 125.73 96.52) (width 0.4) (layer B.Cu) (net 10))
 (segment (start 176.53 97.79) (end 176.53 91.44) (width 0.4) (layer B.Cu) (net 10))
 (segment (start 176.53 91.44) (end 182.88 85.09) (width 0.4) (layer B.Cu) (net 10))
 (segment (start 182.88 85.09) (end 182.88 74.93) (width 0.4) (layer B.Cu) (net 10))
 (segment (start 173.99 66.04) (end 153.67 66.04) (width 0.4) (layer B.Cu) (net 10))
 (segment (start 182.88 74.93) (end 173.99 66.04) (width 0.4) (layer B.Cu) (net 10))
 (segment (start 115.57 66.04) (end 115.57 63.5) (width 0.4) (layer B.Cu) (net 10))
 (segment (start 115.57 63.5) (end 114.3 62.23) (width 0.4) (layer B.Cu) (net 10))
 (segment (start 114.3 62.23) (end 95.25 62.23) (width 0.4) (layer B.Cu) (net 10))
 (segment (start 95.25 62.23) (end 91.44 66.04) (width 0.4) (layer B.Cu) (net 10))
 (segment (start 91.44 68.58) (end 91.44 66.04) (width 0.4) (layer B.Cu) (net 10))
 (segment (start 91.44 68.58) (end 85.09 68.58) (width 0.4) (layer B.Cu) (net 10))
 (segment (start 125.73 66.04) (end 125.73 63.5) (width 0.4) (layer B.Cu) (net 10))
 (segment (start 125.73 63.5) (end 124.46 62.23) (width 0.4) (layer B.Cu) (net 10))
 (segment (start 124.46 62.23) (end 114.3 62.23) (width 0.4) (layer B.Cu) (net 10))
 (segment (start 153.67 63.5) (end 153.67 66.04) (width 0.4) (layer B.Cu) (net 10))
 (segment (start 152.4 62.23) (end 153.67 63.5) (width 0.4) (layer B.Cu) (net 10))
 (segment (start 124.46 62.23) (end 152.4 62.23) (width 0.4) (layer B.Cu) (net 10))
 (segment (start 168.91 74.93) (end 168.91 66.04) (width 0.4) (layer F.Cu) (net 4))
 (segment (start 168.91 66.04) (end 165.1 62.23) (width 0.4) (layer F.Cu) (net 4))
 (segment (start 165.1 62.23) (end 142.24 62.23) (width 0.4) (layer F.Cu) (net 4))
 (segment (start 140.97 63.5) (end 140.97 66.04) (width 0.4) (layer F.Cu) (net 4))
 (segment (start 142.24 62.23) (end 140.97 63.5) (width 0.4) (layer F.Cu) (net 4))
 (segment (start 171.45 74.93) (end 171.45 66.04) (width 0.4) (layer F.Cu) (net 5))
 (segment (start 128.27 63.5) (end 128.27 66.04) (width 0.4) (layer F.Cu) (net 5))
 (segment (start 166.37 60.96) (end 130.81 60.96) (width 0.4) (layer F.Cu) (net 5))
 (segment (start 130.81 60.96) (end 128.27 63.5) (width 0.4) (layer F.Cu) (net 5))
 (segment (start 171.45 66.04) (end 166.37 60.96) (width 0.4) (layer F.Cu) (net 5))
 (segment (start 173.99 74.93) (end 173.99 66.04) (width 0.4) (layer F.Cu) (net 6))
 (segment (start 123.19 63.5) (end 127 59.69) (width 0.4) (layer F.Cu) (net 6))
 (segment (start 123.19 63.5) (end 123.19 66.04) (width 0.4) (layer F.Cu) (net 6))
 (segment (start 127 59.69) (end 167.64 59.69) (width 0.4) (layer F.Cu) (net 6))
 (segment (start 173.99 66.04) (end 167.64 59.69) (width 0.4) (layer F.Cu) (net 6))
 (segment (start 148.59 66.04) (end 148.59 71.12) (width 0.4) (layer F.Cu) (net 12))
 (segment (start 171.45 95.25) (end 148.59 72.39) (width 0.4) (layer F.Cu) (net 12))
 (segment (start 171.45 95.25) (end 171.45 97.79) (width 0.4) (layer F.Cu) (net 12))
 (segment (start 148.59 72.39) (end 148.59 71.12) (width 0.4) (layer F.Cu) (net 12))
 (segment (start 146.05 72.39) (end 146.05 71.12) (width 0.4) (layer F.Cu) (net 13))
 (segment (start 168.91 95.25) (end 146.05 72.39) (width 0.4) (layer F.Cu) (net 13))
 (segment (start 146.05 71.12) (end 146.05 66.04) (width 0.4) (layer F.Cu) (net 13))
 (segment (start 168.91 97.79) (end 168.91 95.25) (width 0.4) (layer F.Cu) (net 13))
 (segment (start 143.51 72.39) (end 143.51 66.04) (width 0.4) (layer F.Cu) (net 14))
 (segment (start 166.37 95.25) (end 143.51 72.39) (width 0.4) (layer F.Cu) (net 14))
 (segment (start 166.37 97.79) (end 166.37 95.25) (width 0.4) (layer F.Cu) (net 14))
 (segment (start 85.09 82.55) (end 90.17 87.63) (width 0.4) (layer B.Cu) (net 7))
 (segment (start 85.09 78.74) (end 85.09 82.55) (width 0.4) (layer B.Cu) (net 7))
 (segment (start 176.53 77.47) (end 176.53 74.93) (width 0.4) (layer B.Cu) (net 7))
 (segment (start 166.37 87.63) (end 176.53 77.47) (width 0.4) (layer B.Cu) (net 7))
 (segment (start 90.17 87.63) (end 166.37 87.63) (width 0.4) (layer B.Cu) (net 7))
 (segment (start 125.73 82.55) (end 125.73 78.74) (width 0.4) (layer F.Cu) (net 22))
 (segment (start 120.65 73.66) (end 120.65 66.04) (width 0.4) (layer F.Cu) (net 22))
 (segment (start 125.73 78.74) (end 120.65 73.66) (width 0.4) (layer F.Cu) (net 22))
 (segment (start 120.65 82.55) (end 120.65 73.66) (width 0.4) (layer F.Cu) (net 22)))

